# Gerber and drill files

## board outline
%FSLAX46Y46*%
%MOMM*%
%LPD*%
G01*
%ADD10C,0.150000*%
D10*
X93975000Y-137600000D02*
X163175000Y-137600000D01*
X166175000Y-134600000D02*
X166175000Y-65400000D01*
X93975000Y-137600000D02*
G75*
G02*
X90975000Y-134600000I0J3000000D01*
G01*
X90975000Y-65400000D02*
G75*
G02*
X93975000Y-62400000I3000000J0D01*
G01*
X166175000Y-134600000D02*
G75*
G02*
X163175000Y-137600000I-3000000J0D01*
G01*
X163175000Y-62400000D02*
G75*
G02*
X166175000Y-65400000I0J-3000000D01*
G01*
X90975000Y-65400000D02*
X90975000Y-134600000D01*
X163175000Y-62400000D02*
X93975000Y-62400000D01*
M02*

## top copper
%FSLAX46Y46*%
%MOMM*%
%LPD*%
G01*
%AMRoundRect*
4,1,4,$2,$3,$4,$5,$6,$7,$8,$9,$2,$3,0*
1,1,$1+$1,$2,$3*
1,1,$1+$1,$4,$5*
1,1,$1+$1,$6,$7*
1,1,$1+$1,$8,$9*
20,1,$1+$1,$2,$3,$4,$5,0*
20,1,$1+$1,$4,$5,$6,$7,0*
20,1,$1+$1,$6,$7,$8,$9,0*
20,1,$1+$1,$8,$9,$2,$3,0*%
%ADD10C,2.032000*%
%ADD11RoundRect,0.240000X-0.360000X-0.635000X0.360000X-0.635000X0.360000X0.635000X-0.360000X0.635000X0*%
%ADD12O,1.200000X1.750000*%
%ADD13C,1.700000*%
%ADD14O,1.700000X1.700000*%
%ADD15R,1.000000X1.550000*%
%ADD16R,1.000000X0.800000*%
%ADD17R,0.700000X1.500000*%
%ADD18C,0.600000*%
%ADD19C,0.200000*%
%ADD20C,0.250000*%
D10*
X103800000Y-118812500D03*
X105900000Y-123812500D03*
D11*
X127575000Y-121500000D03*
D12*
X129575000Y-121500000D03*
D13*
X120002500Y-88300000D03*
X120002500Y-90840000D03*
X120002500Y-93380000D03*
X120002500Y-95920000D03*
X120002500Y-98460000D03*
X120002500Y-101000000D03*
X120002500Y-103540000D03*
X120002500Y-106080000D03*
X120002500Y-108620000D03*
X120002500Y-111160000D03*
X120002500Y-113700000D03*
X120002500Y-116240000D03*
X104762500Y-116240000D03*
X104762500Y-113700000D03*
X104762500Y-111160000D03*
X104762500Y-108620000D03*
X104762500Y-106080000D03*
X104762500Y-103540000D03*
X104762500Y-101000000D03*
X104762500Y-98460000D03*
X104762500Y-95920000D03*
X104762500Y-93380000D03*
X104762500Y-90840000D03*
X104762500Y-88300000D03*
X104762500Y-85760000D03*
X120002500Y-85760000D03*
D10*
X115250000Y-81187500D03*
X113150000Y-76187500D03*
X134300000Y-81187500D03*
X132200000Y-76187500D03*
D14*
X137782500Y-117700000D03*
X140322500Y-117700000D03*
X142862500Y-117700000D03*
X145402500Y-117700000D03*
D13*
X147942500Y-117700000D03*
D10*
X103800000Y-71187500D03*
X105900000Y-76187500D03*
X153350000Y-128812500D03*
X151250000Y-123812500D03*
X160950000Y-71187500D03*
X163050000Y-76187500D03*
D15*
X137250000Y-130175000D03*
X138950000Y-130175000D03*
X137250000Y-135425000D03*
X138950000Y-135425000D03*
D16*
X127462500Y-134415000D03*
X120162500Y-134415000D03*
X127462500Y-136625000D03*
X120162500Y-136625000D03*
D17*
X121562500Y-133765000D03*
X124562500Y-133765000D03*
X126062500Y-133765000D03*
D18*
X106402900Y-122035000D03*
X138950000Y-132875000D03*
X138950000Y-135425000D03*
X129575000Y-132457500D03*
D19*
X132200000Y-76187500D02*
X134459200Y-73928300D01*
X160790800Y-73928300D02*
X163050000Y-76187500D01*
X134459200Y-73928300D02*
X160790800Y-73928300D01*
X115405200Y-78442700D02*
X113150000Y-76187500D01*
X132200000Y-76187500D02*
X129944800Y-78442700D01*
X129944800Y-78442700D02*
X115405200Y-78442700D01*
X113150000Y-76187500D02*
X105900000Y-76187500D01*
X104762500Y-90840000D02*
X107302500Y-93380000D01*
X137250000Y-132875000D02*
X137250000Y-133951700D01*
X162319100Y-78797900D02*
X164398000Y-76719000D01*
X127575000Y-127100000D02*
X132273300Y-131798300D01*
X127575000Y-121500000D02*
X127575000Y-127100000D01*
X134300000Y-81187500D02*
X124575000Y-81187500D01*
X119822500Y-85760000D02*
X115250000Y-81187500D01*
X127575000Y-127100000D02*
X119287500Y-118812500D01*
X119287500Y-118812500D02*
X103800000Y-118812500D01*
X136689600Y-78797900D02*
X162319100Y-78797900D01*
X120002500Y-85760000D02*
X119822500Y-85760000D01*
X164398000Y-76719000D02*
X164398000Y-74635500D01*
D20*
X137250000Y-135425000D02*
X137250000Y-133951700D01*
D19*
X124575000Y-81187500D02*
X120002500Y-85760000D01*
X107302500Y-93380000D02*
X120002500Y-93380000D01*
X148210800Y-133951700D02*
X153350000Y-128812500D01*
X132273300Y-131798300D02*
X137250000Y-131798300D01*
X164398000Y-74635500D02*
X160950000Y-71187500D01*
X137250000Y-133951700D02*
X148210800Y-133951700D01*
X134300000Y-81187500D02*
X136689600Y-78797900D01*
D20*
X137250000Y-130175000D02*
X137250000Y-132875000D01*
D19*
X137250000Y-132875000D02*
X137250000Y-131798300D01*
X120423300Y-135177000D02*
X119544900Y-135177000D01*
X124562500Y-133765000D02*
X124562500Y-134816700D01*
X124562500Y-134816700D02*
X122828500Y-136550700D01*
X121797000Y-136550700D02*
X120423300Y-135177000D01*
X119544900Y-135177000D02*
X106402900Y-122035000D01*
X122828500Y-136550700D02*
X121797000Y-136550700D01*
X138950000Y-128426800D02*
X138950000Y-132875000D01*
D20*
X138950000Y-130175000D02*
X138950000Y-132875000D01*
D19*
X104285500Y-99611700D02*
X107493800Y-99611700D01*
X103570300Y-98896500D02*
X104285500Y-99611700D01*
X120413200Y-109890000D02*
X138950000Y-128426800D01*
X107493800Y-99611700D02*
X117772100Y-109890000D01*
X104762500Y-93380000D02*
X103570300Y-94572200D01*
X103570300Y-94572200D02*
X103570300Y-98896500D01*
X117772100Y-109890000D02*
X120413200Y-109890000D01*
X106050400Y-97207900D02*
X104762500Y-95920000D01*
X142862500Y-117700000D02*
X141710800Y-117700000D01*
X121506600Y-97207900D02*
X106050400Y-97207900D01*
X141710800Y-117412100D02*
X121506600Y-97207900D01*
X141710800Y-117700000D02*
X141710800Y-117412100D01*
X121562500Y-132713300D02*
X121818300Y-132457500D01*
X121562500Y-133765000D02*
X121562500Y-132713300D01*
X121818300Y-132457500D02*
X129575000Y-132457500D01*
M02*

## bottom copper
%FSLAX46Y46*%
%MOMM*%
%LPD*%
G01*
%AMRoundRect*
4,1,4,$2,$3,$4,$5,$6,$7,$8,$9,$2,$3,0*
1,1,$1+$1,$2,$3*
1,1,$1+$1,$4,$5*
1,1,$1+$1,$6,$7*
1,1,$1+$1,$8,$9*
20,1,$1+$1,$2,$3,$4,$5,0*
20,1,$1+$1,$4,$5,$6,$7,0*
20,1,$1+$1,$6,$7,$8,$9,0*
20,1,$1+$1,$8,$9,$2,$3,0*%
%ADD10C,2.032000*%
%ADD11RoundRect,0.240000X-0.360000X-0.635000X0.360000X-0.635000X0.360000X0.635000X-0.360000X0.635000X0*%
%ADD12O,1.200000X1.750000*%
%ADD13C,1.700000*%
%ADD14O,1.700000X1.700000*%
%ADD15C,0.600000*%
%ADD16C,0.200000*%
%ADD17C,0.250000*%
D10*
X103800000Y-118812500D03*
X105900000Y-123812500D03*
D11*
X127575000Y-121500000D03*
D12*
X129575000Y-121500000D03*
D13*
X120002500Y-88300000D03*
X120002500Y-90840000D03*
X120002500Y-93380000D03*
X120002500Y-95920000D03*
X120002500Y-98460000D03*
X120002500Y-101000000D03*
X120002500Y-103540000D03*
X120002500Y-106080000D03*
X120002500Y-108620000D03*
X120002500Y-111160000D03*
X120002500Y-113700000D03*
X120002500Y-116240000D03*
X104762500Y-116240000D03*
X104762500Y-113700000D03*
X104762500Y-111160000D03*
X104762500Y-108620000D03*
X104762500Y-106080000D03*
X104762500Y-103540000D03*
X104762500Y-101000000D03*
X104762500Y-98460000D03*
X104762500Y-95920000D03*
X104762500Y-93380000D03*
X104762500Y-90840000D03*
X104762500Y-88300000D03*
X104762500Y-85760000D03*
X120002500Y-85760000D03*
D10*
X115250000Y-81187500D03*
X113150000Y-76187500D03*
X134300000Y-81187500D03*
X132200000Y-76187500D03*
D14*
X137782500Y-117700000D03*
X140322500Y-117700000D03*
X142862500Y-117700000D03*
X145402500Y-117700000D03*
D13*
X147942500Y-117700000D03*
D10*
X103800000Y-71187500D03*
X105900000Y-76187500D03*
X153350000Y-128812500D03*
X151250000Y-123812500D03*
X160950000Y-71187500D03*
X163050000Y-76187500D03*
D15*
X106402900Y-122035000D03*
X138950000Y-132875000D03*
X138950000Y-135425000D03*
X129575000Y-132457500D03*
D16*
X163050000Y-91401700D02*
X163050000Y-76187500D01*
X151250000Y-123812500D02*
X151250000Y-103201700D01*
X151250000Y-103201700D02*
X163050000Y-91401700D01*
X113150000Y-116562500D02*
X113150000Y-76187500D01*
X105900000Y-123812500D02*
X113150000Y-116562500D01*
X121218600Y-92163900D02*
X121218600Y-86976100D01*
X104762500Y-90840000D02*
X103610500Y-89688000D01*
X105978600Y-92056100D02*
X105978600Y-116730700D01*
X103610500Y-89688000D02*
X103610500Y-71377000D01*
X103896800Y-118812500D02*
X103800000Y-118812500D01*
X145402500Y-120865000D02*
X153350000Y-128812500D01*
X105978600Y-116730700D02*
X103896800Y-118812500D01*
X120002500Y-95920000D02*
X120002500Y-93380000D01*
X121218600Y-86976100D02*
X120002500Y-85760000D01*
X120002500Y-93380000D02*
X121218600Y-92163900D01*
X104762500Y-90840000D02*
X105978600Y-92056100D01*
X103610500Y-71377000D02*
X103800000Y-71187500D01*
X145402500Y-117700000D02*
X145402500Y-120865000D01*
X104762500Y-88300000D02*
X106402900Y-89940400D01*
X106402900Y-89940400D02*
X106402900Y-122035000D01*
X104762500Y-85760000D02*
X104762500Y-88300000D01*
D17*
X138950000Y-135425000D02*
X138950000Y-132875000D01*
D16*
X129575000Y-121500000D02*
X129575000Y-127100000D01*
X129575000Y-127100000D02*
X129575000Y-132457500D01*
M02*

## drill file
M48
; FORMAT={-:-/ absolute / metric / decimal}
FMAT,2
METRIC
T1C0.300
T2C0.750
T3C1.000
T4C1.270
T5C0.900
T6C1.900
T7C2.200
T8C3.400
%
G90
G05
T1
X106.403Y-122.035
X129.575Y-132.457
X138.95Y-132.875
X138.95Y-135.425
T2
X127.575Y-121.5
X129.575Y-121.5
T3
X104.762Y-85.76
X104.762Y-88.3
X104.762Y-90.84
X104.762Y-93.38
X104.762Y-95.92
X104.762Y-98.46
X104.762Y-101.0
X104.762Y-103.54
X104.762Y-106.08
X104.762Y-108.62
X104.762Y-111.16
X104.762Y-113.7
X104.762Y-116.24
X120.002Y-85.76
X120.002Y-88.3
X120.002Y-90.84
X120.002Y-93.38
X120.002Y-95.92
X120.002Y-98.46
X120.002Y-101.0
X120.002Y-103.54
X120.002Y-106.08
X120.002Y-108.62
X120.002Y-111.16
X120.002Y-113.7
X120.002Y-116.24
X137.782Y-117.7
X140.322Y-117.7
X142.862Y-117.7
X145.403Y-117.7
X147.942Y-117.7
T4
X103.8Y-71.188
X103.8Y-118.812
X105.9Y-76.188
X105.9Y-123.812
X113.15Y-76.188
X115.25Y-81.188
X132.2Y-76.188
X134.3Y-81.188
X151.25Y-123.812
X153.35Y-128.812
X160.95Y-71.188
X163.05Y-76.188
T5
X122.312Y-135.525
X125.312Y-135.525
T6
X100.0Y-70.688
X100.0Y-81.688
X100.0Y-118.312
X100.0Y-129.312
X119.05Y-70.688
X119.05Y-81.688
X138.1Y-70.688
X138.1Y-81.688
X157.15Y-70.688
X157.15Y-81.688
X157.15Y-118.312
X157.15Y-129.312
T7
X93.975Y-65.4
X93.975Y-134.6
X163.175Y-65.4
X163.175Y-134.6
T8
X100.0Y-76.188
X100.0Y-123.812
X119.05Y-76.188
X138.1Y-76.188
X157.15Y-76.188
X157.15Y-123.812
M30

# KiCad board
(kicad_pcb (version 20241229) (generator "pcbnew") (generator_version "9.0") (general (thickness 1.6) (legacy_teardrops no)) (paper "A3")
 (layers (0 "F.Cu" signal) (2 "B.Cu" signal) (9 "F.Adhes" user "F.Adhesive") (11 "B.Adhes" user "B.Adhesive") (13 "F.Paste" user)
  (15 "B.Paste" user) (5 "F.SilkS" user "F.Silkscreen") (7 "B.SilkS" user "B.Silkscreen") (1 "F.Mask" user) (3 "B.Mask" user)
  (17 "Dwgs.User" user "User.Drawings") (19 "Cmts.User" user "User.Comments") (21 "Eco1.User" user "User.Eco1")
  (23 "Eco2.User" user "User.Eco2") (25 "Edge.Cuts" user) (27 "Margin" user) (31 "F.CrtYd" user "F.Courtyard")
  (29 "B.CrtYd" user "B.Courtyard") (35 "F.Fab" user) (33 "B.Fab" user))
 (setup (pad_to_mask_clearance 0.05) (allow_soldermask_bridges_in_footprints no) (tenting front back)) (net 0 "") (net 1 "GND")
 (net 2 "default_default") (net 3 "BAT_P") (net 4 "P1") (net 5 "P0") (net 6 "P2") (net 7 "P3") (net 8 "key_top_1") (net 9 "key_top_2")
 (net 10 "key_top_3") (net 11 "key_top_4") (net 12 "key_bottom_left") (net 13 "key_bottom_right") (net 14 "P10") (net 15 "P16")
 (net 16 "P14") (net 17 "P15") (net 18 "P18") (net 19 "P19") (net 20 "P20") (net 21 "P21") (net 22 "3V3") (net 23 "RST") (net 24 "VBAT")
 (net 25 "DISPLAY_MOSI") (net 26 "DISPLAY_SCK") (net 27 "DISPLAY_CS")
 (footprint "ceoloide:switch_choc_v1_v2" (layer "F.Cu") (at 100 123.8125 -90)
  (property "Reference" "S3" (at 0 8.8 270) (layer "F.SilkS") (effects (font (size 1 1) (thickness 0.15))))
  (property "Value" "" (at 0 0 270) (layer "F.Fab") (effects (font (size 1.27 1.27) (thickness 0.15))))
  (pad "" np_thru_hole circle (at -5.5 0 270) (size 1.9 1.9) (drill 1.9) (layers "*.Cu" "*.Mask"))
  (pad "" np_thru_hole circle (at 0 0 270) (size 3.4 3.4) (drill 3.4) (layers "*.Cu" "*.Mask"))
  (pad "" np_thru_hole circle (at 5.5 0 270) (size 1.9 1.9) (drill 1.9) (layers "*.Cu" "*.Mask"))
  (pad "1" thru_hole circle (at -5 -3.8 105) (size 2.032 2.032) (drill 1.27) (layers "*.Cu" "*.Mask") (remove_unused_layers no)
   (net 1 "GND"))
  (pad "2" thru_hole circle (at 0 -5.9 105) (size 2.032 2.032) (drill 1.27) (layers "*.Cu" "*.Mask") (remove_unused_layers no)
   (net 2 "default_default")))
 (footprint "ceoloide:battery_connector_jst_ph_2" (layer "F.Cu") (at 128.575 121.5)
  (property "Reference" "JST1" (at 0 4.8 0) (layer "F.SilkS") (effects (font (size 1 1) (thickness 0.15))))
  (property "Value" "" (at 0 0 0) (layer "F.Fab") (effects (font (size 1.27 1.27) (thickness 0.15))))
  (pad "1" thru_hole roundrect (at -1 0) (size 1.2 1.75) (drill 0.75) (layers "*.Cu" "*.Mask") (remove_unused_layers no)
   (roundrect_rratio 0.2) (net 1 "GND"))
  (pad "2" thru_hole oval (at 1 0) (size 1.2 1.75) (drill 0.75) (layers "*.Cu" "*.Mask") (remove_unused_layers no) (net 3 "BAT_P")))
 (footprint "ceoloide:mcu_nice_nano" (layer "F.Cu") (at 112.3825 101)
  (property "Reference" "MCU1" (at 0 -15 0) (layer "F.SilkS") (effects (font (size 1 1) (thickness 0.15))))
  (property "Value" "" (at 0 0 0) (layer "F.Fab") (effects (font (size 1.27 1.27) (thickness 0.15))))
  (pad "1" thru_hole circle (at 7.62 -12.7) (size 1.7 1.7) (drill 1) (layers "*.Cu" "*.Mask") (remove_unused_layers no) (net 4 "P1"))
  (pad "2" thru_hole circle (at 7.62 -10.16) (size 1.7 1.7) (drill 1) (layers "*.Cu" "*.Mask") (remove_unused_layers no) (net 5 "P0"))
  (pad "3" thru_hole circle (at 7.62 -7.62) (size 1.7 1.7) (drill 1) (layers "*.Cu" "*.Mask") (remove_unused_layers no) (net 1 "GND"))
  (pad "4" thru_hole circle (at 7.62 -5.08) (size 1.7 1.7) (drill 1) (layers "*.Cu" "*.Mask") (remove_unused_layers no) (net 1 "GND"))
  (pad "5" thru_hole circle (at 7.62 -2.54) (size 1.7 1.7) (drill 1) (layers "*.Cu" "*.Mask") (remove_unused_layers no) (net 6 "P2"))
  (pad "6" thru_hole circle (at 7.62 0) (size 1.7 1.7) (drill 1) (layers "*.Cu" "*.Mask") (remove_unused_layers no) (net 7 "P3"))
  (pad "7" thru_hole circle (at 7.62 2.54) (size 1.7 1.7) (drill 1) (layers "*.Cu" "*.Mask") (remove_unused_layers no) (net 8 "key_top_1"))
  (pad "8" thru_hole circle (at 7.62 5.08) (size 1.7 1.7) (drill 1) (layers "*.Cu" "*.Mask") (remove_unused_layers no) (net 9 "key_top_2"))
  (pad "9" thru_hole circle (at 7.62 7.62) (size 1.7 1.7) (drill 1) (layers "*.Cu" "*.Mask") (remove_unused_layers no) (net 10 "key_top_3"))
  (pad "10" thru_hole circle (at 7.62 10.16) (size 1.7 1.7) (drill 1) (layers "*.Cu" "*.Mask") (remove_unused_layers no)
   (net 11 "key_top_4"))
  (pad "11" thru_hole circle (at 7.62 12.7) (size 1.7 1.7) (drill 1) (layers "*.Cu" "*.Mask") (remove_unused_layers no)
   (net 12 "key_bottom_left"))
  (pad "12" thru_hole circle (at 7.62 15.24) (size 1.7 1.7) (drill 1) (layers "*.Cu" "*.Mask") (remove_unused_layers no)
   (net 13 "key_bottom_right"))
  (pad "13" thru_hole circle (at -7.62 15.24) (size 1.7 1.7) (drill 1) (layers "*.Cu" "*.Mask") (remove_unused_layers no) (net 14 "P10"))
  (pad "14" thru_hole circle (at -7.62 12.7) (size 1.7 1.7) (drill 1) (layers "*.Cu" "*.Mask") (remove_unused_layers no) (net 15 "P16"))
  (pad "15" thru_hole circle (at -7.62 10.16) (size 1.7 1.7) (drill 1) (layers "*.Cu" "*.Mask") (remove_unused_layers no) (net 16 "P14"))
  (pad "16" thru_hole circle (at -7.62 7.62) (size 1.7 1.7) (drill 1) (layers "*.Cu" "*.Mask") (remove_unused_layers no) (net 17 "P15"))
  (pad "17" thru_hole circle (at -7.62 5.08) (size 1.7 1.7) (drill 1) (layers "*.Cu" "*.Mask") (remove_unused_layers no) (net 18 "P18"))
  (pad "18" thru_hole circle (at -7.62 2.54) (size 1.7 1.7) (drill 1) (layers "*.Cu" "*.Mask") (remove_unused_layers no) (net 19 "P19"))
  (pad "19" thru_hole circle (at -7.62 0) (size 1.7 1.7) (drill 1) (layers "*.Cu" "*.Mask") (remove_unused_layers no) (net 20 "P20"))
  (pad "20" thru_hole circle (at -7.62 -2.54) (size 1.7 1.7) (drill 1) (layers "*.Cu" "*.Mask") (remove_unused_layers no) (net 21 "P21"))
  (pad "21" thru_hole circle (at -7.62 -5.08) (size 1.7 1.7) (drill 1) (layers "*.Cu" "*.Mask") (remove_unused_layers no) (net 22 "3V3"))
  (pad "22" thru_hole circle (at -7.62 -7.62) (size 1.7 1.7) (drill 1) (layers "*.Cu" "*.Mask") (remove_unused_layers no) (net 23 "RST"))
  (pad "23" thru_hole circle (at -7.62 -10.16) (size 1.7 1.7) (drill 1) (layers "*.Cu" "*.Mask") (remove_unused_layers no) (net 1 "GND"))
  (pad "24" thru_hole circle (at -7.62 -12.7) (size 1.7 1.7) (drill 1) (layers "*.Cu" "*.Mask") (remove_unused_layers no) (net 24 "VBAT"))
  (pad "25" thru_hole circle (at -7.62 -15.24) (size 1.7 1.7) (drill 1) (layers "*.Cu" "*.Mask") (remove_unused_layers no) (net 24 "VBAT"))
  (pad "26" thru_hole circle (at 7.62 -15.24) (size 1.7 1.7) (drill 1) (layers "*.Cu" "*.Mask") (remove_unused_layers no) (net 1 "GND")))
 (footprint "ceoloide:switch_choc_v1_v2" (layer "F.Cu") (at 119.05 76.1875 90)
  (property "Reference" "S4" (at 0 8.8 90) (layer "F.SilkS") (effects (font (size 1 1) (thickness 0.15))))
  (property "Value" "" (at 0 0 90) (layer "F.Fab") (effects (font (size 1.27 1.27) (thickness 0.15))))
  (pad "" np_thru_hole circle (at -5.5 0 90) (size 1.9 1.9) (drill 1.9) (layers "*.Cu" "*.Mask"))
  (pad "" np_thru_hole circle (at 0 0 90) (size 3.4 3.4) (drill 3.4) (layers "*.Cu" "*.Mask"))
  (pad "" np_thru_hole circle (at 5.5 0 90) (size 1.9 1.9) (drill 1.9) (layers "*.Cu" "*.Mask"))
  (pad "1" thru_hole circle (at -5 -3.8 285) (size 2.032 2.032) (drill 1.27) (layers "*.Cu" "*.Mask") (remove_unused_layers no)
   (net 1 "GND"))
  (pad "2" thru_hole circle (at 0 -5.9 285) (size 2.032 2.032) (drill 1.27) (layers "*.Cu" "*.Mask") (remove_unused_layers no)
   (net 2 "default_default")))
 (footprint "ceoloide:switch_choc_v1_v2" (layer "F.Cu") (at 138.1 76.1875 90)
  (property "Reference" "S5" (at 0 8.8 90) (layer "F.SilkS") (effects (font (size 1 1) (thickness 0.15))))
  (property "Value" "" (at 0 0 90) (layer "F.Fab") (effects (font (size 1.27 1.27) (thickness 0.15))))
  (pad "" np_thru_hole circle (at -5.5 0 90) (size 1.9 1.9) (drill 1.9) (layers "*.Cu" "*.Mask"))
  (pad "" np_thru_hole circle (at 0 0 90) (size 3.4 3.4) (drill 3.4) (layers "*.Cu" "*.Mask"))
  (pad "" np_thru_hole circle (at 5.5 0 90) (size 1.9 1.9) (drill 1.9) (layers "*.Cu" "*.Mask"))
  (pad "1" thru_hole circle (at -5 -3.8 285) (size 2.032 2.032) (drill 1.27) (layers "*.Cu" "*.Mask") (remove_unused_layers no)
   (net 1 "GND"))
  (pad "2" thru_hole circle (at 0 -5.9 285) (size 2.032 2.032) (drill 1.27) (layers "*.Cu" "*.Mask") (remove_unused_layers no)
   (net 2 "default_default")))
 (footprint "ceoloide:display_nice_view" (layer "F.Cu") (at 142.8625 101)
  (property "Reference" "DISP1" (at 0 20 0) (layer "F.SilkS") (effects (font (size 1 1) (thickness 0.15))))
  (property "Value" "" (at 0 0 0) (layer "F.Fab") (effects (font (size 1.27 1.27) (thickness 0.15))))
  (pad "1" thru_hole oval (at -5.08 16.7 270) (size 1.7 1.7) (drill 1) (layers "*.Cu" "*.Mask") (remove_unused_layers no)
   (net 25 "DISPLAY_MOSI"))
  (pad "2" thru_hole oval (at -2.54 16.7 270) (size 1.7 1.7) (drill 1) (layers "*.Cu" "*.Mask") (remove_unused_layers no)
   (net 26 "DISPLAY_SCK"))
  (pad "3" thru_hole oval (at 0 16.7 270) (size 1.7 1.7) (drill 1) (layers "*.Cu" "*.Mask") (remove_unused_layers no) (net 22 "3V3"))
  (pad "4" thru_hole oval (at 2.54 16.7 270) (size 1.7 1.7) (drill 1) (layers "*.Cu" "*.Mask") (remove_unused_layers no) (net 1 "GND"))
  (pad "5" thru_hole circle (at 5.08 16.7 270) (size 1.7 1.7) (drill 1) (layers "*.Cu" "*.Mask") (remove_unused_layers no)
   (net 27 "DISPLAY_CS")))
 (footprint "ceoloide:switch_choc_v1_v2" (layer "F.Cu") (at 100 76.1875 -90)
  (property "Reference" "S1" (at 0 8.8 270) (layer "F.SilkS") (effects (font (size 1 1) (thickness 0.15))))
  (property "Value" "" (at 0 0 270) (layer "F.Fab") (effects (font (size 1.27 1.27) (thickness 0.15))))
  (pad "" np_thru_hole circle (at -5.5 0 270) (size 1.9 1.9) (drill 1.9) (layers "*.Cu" "*.Mask"))
  (pad "" np_thru_hole circle (at 0 0 270) (size 3.4 3.4) (drill 3.4) (layers "*.Cu" "*.Mask"))
  (pad "" np_thru_hole circle (at 5.5 0 270) (size 1.9 1.9) (drill 1.9) (layers "*.Cu" "*.Mask"))
  (pad "1" thru_hole circle (at -5 -3.8 105) (size 2.032 2.032) (drill 1.27) (layers "*.Cu" "*.Mask") (remove_unused_layers no)
   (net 1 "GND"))
  (pad "2" thru_hole circle (at 0 -5.9 105) (size 2.032 2.032) (drill 1.27) (layers "*.Cu" "*.Mask") (remove_unused_layers no)
   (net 2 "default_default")))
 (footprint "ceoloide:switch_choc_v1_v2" (layer "F.Cu") (at 157.15 123.8125 90)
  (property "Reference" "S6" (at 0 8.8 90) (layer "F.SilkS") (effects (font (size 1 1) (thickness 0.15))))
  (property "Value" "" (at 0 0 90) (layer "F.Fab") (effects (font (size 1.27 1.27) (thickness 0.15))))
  (pad "" np_thru_hole circle (at -5.5 0 90) (size 1.9 1.9) (drill 1.9) (layers "*.Cu" "*.Mask"))
  (pad "" np_thru_hole circle (at 0 0 90) (size 3.4 3.4) (drill 3.4) (layers "*.Cu" "*.Mask"))
  (pad "" np_thru_hole circle (at 5.5 0 90) (size 1.9 1.9) (drill 1.9) (layers "*.Cu" "*.Mask"))
  (pad "1" thru_hole circle (at -5 -3.8 285) (size 2.032 2.032) (drill 1.27) (layers "*.Cu" "*.Mask") (remove_unused_layers no)
   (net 1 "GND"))
  (pad "2" thru_hole circle (at 0 -5.9 285) (size 2.032 2.032) (drill 1.27) (layers "*.Cu" "*.Mask") (remove_unused_layers no)
   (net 2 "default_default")))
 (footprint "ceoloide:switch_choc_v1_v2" (layer "F.Cu") (at 157.15 76.1875 -90)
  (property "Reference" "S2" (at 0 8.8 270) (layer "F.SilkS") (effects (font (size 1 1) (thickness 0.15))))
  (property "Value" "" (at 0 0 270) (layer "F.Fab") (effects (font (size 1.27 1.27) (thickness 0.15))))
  (pad "" np_thru_hole circle (at -5.5 0 270) (size 1.9 1.9) (drill 1.9) (layers "*.Cu" "*.Mask"))
  (pad "" np_thru_hole circle (at 0 0 270) (size 3.4 3.4) (drill 3.4) (layers "*.Cu" "*.Mask"))
  (pad "" np_thru_hole circle (at 5.5 0 270) (size 1.9 1.9) (drill 1.9) (layers "*.Cu" "*.Mask"))
  (pad "1" thru_hole circle (at -5 -3.8 105) (size 2.032 2.032) (drill 1.27) (layers "*.Cu" "*.Mask") (remove_unused_layers no)
   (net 1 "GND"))
  (pad "2" thru_hole circle (at 0 -5.9 105) (size 2.032 2.032) (drill 1.27) (layers "*.Cu" "*.Mask") (remove_unused_layers no)
   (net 2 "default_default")))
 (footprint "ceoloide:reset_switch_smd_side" (layer "F.Cu") (at 138.1 132.8 90)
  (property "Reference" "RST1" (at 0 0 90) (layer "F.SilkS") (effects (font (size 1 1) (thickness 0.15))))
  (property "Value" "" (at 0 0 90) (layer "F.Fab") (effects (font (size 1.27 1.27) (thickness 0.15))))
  (pad "1" smd rect (at 2.625 -0.85 270) (size 1.55 1) (layers "F.Cu" "F.Mask" "F.Paste") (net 1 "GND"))
  (pad "2" smd rect (at 2.625 0.85 270) (size 1.55 1) (layers "F.Cu" "F.Mask" "F.Paste") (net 23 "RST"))
  (pad "3" smd rect (at -2.625 -0.85 270) (size 1.55 1) (layers "F.Cu" "F.Mask" "F.Paste") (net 1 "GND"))
  (pad "4" smd rect (at -2.625 0.85 270) (size 1.55 1) (layers "F.Cu" "F.Mask" "F.Paste") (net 23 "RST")))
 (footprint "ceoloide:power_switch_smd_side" (layer "F.Cu") (at 123.8125 135.5 -90)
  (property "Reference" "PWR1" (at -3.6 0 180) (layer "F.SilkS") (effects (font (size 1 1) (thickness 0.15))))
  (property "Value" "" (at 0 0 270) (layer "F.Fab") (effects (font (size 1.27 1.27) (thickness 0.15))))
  (pad "" smd rect (at -1.085 -3.65) (size 1 0.8) (layers "F.Cu" "F.Mask" "F.Paste"))
  (pad "" smd rect (at -1.085 3.65) (size 1 0.8) (layers "F.Cu" "F.Mask" "F.Paste"))
  (pad "" np_thru_hole circle (at 0.025 -1.5) (size 0.9 0.9) (drill 0.9) (layers "*.Cu" "*.Mask"))
  (pad "" np_thru_hole circle (at 0.025 1.5) (size 0.9 0.9) (drill 0.9) (layers "*.Cu" "*.Mask"))
  (pad "" smd rect (at 1.125 -3.65) (size 1 0.8) (layers "F.Cu" "F.Mask" "F.Paste"))
  (pad "" smd rect (at 1.125 3.65) (size 1 0.8) (layers "F.Cu" "F.Mask" "F.Paste"))
  (pad "1" smd rect (at -1.735 2.25) (size 0.7 1.5) (layers "F.Cu" "F.Mask" "F.Paste") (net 3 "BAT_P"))
  (pad "2" smd rect (at -1.735 -0.75) (size 0.7 1.5) (layers "F.Cu" "F.Mask" "F.Paste") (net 24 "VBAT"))
  (pad "3" smd rect (at -1.735 -2.25) (size 0.7 1.5) (layers "F.Cu" "F.Mask" "F.Paste")))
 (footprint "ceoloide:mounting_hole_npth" (layer "B.Cu") (at 93.975 134.6)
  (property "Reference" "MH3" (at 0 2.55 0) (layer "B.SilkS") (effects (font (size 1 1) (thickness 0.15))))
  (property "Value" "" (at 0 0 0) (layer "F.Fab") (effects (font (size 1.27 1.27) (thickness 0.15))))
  (pad "" np_thru_hole circle (at 0 0) (size 2.2 2.2) (drill 2.2) (layers "*.Cu" "*.Mask")))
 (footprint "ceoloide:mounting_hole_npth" (layer "B.Cu") (at 93.975 65.4)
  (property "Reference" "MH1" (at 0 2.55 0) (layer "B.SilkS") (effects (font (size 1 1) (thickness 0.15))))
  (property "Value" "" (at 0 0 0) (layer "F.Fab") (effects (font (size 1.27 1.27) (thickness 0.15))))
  (pad "" np_thru_hole circle (at 0 0) (size 2.2 2.2) (drill 2.2) (layers "*.Cu" "*.Mask")))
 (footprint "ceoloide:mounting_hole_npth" (layer "B.Cu") (at 163.175 134.6)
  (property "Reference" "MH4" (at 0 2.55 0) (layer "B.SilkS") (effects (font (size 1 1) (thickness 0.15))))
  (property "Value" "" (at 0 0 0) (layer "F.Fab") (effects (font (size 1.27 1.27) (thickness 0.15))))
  (pad "" np_thru_hole circle (at 0 0) (size 2.2 2.2) (drill 2.2) (layers "*.Cu" "*.Mask")))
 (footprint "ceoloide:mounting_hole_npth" (layer "B.Cu") (at 163.175 65.4)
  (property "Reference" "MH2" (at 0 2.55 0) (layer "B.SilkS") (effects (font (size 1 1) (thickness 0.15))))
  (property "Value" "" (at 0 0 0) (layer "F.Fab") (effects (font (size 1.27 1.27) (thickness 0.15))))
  (pad "" np_thru_hole circle (at 0 0) (size 2.2 2.2) (drill 2.2) (layers "*.Cu" "*.Mask")))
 (gr_line (start 93.975 137.6) (end 163.175 137.6) (stroke (width 0.15) (type default)) (layer "Edge.Cuts"))
 (gr_line (start 166.175 134.6) (end 166.175 65.4) (stroke (width 0.15) (type default)) (layer "Edge.Cuts"))
 (gr_arc (start 93.975 137.6) (mid 91.85368 136.72132) (end 90.975 134.6) (stroke (width 0.15) (type default)) (layer "Edge.Cuts"))
 (gr_arc (start 90.975 65.4) (mid 91.85368 63.27868) (end 93.975 62.4) (stroke (width 0.15) (type default)) (layer "Edge.Cuts"))
 (gr_arc (start 166.175 134.6) (mid 165.29632 136.72132) (end 163.175 137.6) (stroke (width 0.15) (type default)) (layer "Edge.Cuts"))
 (gr_arc (start 163.175 62.4) (mid 165.29632 63.27868) (end 166.175 65.4) (stroke (width 0.15) (type default)) (layer "Edge.Cuts"))
 (gr_line (start 90.975 65.4) (end 90.975 134.6) (stroke (width 0.15) (type default)) (layer "Edge.Cuts"))
 (gr_line (start 163.175 62.4) (end 93.975 62.4) (stroke (width 0.15) (type default)) (layer "Edge.Cuts"))
 (segment (start 132.2 76.1875) (end 134.4592 73.9283) (width 0.2) (layer "F.Cu") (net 2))
 (segment (start 160.7908 73.9283) (end 163.05 76.1875) (width 0.2) (layer "F.Cu") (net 2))
 (segment (start 134.4592 73.9283) (end 160.7908 73.9283) (width 0.2) (layer "F.Cu") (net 2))
 (segment (start 115.4052 78.4427) (end 113.15 76.1875) (width 0.2) (layer "F.Cu") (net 2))
 (segment (start 132.2 76.1875) (end 129.9448 78.4427) (width 0.2) (layer "F.Cu") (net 2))
 (segment (start 129.9448 78.4427) (end 115.4052 78.4427) (width 0.2) (layer "F.Cu") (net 2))
 (segment (start 113.15 76.1875) (end 105.9 76.1875) (width 0.2) (layer "F.Cu") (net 2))
 (segment (start 163.05 91.4017) (end 163.05 76.1875) (width 0.2) (layer "B.Cu") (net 2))
 (segment (start 151.25 123.8125) (end 151.25 103.2017) (width 0.2) (layer "B.Cu") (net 2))
 (segment (start 151.25 103.2017) (end 163.05 91.4017) (width 0.2) (layer "B.Cu") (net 2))
 (segment (start 113.15 116.5625) (end 113.15 76.1875) (width 0.2) (layer "B.Cu") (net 2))
 (segment (start 105.9 123.8125) (end 113.15 116.5625) (width 0.2) (layer "B.Cu") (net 2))
 (segment (start 104.7625 90.84) (end 107.3025 93.38) (width 0.2) (layer "F.Cu") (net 1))
 (segment (start 137.25 132.875) (end 137.25 133.9517) (width 0.2) (layer "F.Cu") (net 1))
 (segment (start 162.3191 78.7979) (end 164.398 76.719) (width 0.2) (layer "F.Cu") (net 1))
 (segment (start 127.575 127.1) (end 132.2733 131.7983) (width 0.2) (layer "F.Cu") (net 1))
 (segment (start 127.575 121.5) (end 127.575 127.1) (width 0.2) (layer "F.Cu") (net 1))
 (segment (start 134.3 81.1875) (end 124.575 81.1875) (width 0.2) (layer "F.Cu") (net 1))
 (segment (start 119.8225 85.76) (end 115.25 81.1875) (width 0.2) (layer "F.Cu") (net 1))
 (segment (start 127.575 127.1) (end 119.2875 118.8125) (width 0.2) (layer "F.Cu") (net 1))
 (segment (start 119.2875 118.8125) (end 103.8 118.8125) (width 0.2) (layer "F.Cu") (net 1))
 (segment (start 136.6896 78.7979) (end 162.3191 78.7979) (width 0.2) (layer "F.Cu") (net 1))
 (segment (start 120.0025 85.76) (end 119.8225 85.76) (width 0.2) (layer "F.Cu") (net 1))
 (segment (start 164.398 76.719) (end 164.398 74.6355) (width 0.2) (layer "F.Cu") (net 1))
 (segment (start 137.25 135.425) (end 137.25 133.9517) (width 0.25) (layer "F.Cu") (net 1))
 (segment (start 124.575 81.1875) (end 120.0025 85.76) (width 0.2) (layer "F.Cu") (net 1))
 (segment (start 107.3025 93.38) (end 120.0025 93.38) (width 0.2) (layer "F.Cu") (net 1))
 (segment (start 148.2108 133.9517) (end 153.35 128.8125) (width 0.2) (layer "F.Cu") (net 1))
 (segment (start 132.2733 131.7983) (end 137.25 131.7983) (width 0.2) (layer "F.Cu") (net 1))
 (segment (start 164.398 74.6355) (end 160.95 71.1875) (width 0.2) (layer "F.Cu") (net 1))
 (segment (start 137.25 133.9517) (end 148.2108 133.9517) (width 0.2) (layer "F.Cu") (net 1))
 (segment (start 134.3 81.1875) (end 136.6896 78.7979) (width 0.2) (layer "F.Cu") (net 1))
 (segment (start 137.25 130.175) (end 137.25 132.875) (width 0.25) (layer "F.Cu") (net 1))
 (segment (start 137.25 132.875) (end 137.25 131.7983) (width 0.2) (layer "F.Cu") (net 1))
 (segment (start 121.2186 92.1639) (end 121.2186 86.9761) (width 0.2) (layer "B.Cu") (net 1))
 (segment (start 104.7625 90.84) (end 103.6105 89.688) (width 0.2) (layer "B.Cu") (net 1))
 (segment (start 105.9786 92.0561) (end 105.9786 116.7307) (width 0.2) (layer "B.Cu") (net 1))
 (segment (start 103.6105 89.688) (end 103.6105 71.377) (width 0.2) (layer "B.Cu") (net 1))
 (segment (start 103.8968 118.8125) (end 103.8 118.8125) (width 0.2) (layer "B.Cu") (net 1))
 (segment (start 145.4025 120.865) (end 153.35 128.8125) (width 0.2) (layer "B.Cu") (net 1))
 (segment (start 105.9786 116.7307) (end 103.8968 118.8125) (width 0.2) (layer "B.Cu") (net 1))
 (segment (start 120.0025 95.92) (end 120.0025 93.38) (width 0.2) (layer "B.Cu") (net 1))
 (segment (start 121.2186 86.9761) (end 120.0025 85.76) (width 0.2) (layer "B.Cu") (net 1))
 (segment (start 120.0025 93.38) (end 121.2186 92.1639) (width 0.2) (layer "B.Cu") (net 1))
 (segment (start 104.7625 90.84) (end 105.9786 92.0561) (width 0.2) (layer "B.Cu") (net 1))
 (segment (start 103.6105 71.377) (end 103.8 71.1875) (width 0.2) (layer "B.Cu") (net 1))
 (segment (start 145.4025 117.7) (end 145.4025 120.865) (width 0.2) (layer "B.Cu") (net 1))
 (segment (start 120.4233 135.177) (end 119.5449 135.177) (width 0.2) (layer "F.Cu") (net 24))
 (segment (start 124.5625 133.765) (end 124.5625 134.8167) (width 0.2) (layer "F.Cu") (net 24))
 (segment (start 124.5625 134.8167) (end 122.8285 136.5507) (width 0.2) (layer "F.Cu") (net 24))
 (segment (start 121.797 136.5507) (end 120.4233 135.177) (width 0.2) (layer "F.Cu") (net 24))
 (segment (start 119.5449 135.177) (end 106.4029 122.035) (width 0.2) (layer "F.Cu") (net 24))
 (segment (start 122.8285 136.5507) (end 121.797 136.5507) (width 0.2) (layer "F.Cu") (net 24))
 (via (at 106.4029 122.035) (size 0.6) (drill 0.3) (layers "F.Cu" "B.Cu") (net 24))
 (segment (start 104.7625 88.3) (end 106.4029 89.9404) (width 0.2) (layer "B.Cu") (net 24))
 (segment (start 106.4029 89.9404) (end 106.4029 122.035) (width 0.2) (layer "B.Cu") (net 24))
 (segment (start 104.7625 85.76) (end 104.7625 88.3) (width 0.2) (layer "B.Cu") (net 24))
 (segment (start 138.95 128.4268) (end 138.95 132.875) (width 0.2) (layer "F.Cu") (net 23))
 (segment (start 138.95 130.175) (end 138.95 132.875) (width 0.25) (layer "F.Cu") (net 23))
 (segment (start 104.2855 99.6117) (end 107.4938 99.6117) (width 0.2) (layer "F.Cu") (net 23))
 (segment (start 103.5703 98.8965) (end 104.2855 99.6117) (width 0.2) (layer "F.Cu") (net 23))
 (segment (start 120.4132 109.89) (end 138.95 128.4268) (width 0.2) (layer "F.Cu") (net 23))
 (segment (start 107.4938 99.6117) (end 117.7721 109.89) (width 0.2) (layer "F.Cu") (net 23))
 (segment (start 104.7625 93.38) (end 103.5703 94.5722) (width 0.2) (layer "F.Cu") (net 23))
 (segment (start 103.5703 94.5722) (end 103.5703 98.8965) (width 0.2) (layer "F.Cu") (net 23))
 (segment (start 117.7721 109.89) (end 120.4132 109.89) (width 0.2) (layer "F.Cu") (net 23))
 (via (at 138.95 132.875) (size 0.6) (drill 0.3) (layers "F.Cu" "B.Cu") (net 23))
 (via (at 138.95 135.425) (size 0.6) (drill 0.3) (layers "F.Cu" "B.Cu") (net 23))
 (segment (start 138.95 135.425) (end 138.95 132.875) (width 0.25) (layer "B.Cu") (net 23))
 (segment (start 106.0504 97.2079) (end 104.7625 95.92) (width 0.2) (layer "F.Cu") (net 22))
 (segment (start 142.8625 117.7) (end 141.7108 117.7) (width 0.2) (layer "F.Cu") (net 22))
 (segment (start 121.5066 97.2079) (end 106.0504 97.2079) (width 0.2) (layer "F.Cu") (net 22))
 (segment (start 141.7108 117.4121) (end 121.5066 97.2079) (width 0.2) (layer "F.Cu") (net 22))
 (segment (start 141.7108 117.7) (end 141.7108 117.4121) (width 0.2) (layer "F.Cu") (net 22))
 (segment (start 121.5625 132.7133) (end 121.8183 132.4575) (width 0.2) (layer "F.Cu") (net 3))
 (segment (start 121.5625 133.765) (end 121.5625 132.7133) (width 0.2) (layer "F.Cu") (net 3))
 (segment (start 121.8183 132.4575) (end 129.575 132.4575) (width 0.2) (layer "F.Cu") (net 3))
 (via (at 129.575 132.4575) (size 0.6) (drill 0.3) (layers "F.Cu" "B.Cu") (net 3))
 (segment (start 129.575 121.5) (end 129.575 127.1) (width 0.2) (layer "B.Cu") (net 3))
 (segment (start 129.575 127.1) (end 129.575 132.4575) (width 0.2) (layer "B.Cu") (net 3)))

